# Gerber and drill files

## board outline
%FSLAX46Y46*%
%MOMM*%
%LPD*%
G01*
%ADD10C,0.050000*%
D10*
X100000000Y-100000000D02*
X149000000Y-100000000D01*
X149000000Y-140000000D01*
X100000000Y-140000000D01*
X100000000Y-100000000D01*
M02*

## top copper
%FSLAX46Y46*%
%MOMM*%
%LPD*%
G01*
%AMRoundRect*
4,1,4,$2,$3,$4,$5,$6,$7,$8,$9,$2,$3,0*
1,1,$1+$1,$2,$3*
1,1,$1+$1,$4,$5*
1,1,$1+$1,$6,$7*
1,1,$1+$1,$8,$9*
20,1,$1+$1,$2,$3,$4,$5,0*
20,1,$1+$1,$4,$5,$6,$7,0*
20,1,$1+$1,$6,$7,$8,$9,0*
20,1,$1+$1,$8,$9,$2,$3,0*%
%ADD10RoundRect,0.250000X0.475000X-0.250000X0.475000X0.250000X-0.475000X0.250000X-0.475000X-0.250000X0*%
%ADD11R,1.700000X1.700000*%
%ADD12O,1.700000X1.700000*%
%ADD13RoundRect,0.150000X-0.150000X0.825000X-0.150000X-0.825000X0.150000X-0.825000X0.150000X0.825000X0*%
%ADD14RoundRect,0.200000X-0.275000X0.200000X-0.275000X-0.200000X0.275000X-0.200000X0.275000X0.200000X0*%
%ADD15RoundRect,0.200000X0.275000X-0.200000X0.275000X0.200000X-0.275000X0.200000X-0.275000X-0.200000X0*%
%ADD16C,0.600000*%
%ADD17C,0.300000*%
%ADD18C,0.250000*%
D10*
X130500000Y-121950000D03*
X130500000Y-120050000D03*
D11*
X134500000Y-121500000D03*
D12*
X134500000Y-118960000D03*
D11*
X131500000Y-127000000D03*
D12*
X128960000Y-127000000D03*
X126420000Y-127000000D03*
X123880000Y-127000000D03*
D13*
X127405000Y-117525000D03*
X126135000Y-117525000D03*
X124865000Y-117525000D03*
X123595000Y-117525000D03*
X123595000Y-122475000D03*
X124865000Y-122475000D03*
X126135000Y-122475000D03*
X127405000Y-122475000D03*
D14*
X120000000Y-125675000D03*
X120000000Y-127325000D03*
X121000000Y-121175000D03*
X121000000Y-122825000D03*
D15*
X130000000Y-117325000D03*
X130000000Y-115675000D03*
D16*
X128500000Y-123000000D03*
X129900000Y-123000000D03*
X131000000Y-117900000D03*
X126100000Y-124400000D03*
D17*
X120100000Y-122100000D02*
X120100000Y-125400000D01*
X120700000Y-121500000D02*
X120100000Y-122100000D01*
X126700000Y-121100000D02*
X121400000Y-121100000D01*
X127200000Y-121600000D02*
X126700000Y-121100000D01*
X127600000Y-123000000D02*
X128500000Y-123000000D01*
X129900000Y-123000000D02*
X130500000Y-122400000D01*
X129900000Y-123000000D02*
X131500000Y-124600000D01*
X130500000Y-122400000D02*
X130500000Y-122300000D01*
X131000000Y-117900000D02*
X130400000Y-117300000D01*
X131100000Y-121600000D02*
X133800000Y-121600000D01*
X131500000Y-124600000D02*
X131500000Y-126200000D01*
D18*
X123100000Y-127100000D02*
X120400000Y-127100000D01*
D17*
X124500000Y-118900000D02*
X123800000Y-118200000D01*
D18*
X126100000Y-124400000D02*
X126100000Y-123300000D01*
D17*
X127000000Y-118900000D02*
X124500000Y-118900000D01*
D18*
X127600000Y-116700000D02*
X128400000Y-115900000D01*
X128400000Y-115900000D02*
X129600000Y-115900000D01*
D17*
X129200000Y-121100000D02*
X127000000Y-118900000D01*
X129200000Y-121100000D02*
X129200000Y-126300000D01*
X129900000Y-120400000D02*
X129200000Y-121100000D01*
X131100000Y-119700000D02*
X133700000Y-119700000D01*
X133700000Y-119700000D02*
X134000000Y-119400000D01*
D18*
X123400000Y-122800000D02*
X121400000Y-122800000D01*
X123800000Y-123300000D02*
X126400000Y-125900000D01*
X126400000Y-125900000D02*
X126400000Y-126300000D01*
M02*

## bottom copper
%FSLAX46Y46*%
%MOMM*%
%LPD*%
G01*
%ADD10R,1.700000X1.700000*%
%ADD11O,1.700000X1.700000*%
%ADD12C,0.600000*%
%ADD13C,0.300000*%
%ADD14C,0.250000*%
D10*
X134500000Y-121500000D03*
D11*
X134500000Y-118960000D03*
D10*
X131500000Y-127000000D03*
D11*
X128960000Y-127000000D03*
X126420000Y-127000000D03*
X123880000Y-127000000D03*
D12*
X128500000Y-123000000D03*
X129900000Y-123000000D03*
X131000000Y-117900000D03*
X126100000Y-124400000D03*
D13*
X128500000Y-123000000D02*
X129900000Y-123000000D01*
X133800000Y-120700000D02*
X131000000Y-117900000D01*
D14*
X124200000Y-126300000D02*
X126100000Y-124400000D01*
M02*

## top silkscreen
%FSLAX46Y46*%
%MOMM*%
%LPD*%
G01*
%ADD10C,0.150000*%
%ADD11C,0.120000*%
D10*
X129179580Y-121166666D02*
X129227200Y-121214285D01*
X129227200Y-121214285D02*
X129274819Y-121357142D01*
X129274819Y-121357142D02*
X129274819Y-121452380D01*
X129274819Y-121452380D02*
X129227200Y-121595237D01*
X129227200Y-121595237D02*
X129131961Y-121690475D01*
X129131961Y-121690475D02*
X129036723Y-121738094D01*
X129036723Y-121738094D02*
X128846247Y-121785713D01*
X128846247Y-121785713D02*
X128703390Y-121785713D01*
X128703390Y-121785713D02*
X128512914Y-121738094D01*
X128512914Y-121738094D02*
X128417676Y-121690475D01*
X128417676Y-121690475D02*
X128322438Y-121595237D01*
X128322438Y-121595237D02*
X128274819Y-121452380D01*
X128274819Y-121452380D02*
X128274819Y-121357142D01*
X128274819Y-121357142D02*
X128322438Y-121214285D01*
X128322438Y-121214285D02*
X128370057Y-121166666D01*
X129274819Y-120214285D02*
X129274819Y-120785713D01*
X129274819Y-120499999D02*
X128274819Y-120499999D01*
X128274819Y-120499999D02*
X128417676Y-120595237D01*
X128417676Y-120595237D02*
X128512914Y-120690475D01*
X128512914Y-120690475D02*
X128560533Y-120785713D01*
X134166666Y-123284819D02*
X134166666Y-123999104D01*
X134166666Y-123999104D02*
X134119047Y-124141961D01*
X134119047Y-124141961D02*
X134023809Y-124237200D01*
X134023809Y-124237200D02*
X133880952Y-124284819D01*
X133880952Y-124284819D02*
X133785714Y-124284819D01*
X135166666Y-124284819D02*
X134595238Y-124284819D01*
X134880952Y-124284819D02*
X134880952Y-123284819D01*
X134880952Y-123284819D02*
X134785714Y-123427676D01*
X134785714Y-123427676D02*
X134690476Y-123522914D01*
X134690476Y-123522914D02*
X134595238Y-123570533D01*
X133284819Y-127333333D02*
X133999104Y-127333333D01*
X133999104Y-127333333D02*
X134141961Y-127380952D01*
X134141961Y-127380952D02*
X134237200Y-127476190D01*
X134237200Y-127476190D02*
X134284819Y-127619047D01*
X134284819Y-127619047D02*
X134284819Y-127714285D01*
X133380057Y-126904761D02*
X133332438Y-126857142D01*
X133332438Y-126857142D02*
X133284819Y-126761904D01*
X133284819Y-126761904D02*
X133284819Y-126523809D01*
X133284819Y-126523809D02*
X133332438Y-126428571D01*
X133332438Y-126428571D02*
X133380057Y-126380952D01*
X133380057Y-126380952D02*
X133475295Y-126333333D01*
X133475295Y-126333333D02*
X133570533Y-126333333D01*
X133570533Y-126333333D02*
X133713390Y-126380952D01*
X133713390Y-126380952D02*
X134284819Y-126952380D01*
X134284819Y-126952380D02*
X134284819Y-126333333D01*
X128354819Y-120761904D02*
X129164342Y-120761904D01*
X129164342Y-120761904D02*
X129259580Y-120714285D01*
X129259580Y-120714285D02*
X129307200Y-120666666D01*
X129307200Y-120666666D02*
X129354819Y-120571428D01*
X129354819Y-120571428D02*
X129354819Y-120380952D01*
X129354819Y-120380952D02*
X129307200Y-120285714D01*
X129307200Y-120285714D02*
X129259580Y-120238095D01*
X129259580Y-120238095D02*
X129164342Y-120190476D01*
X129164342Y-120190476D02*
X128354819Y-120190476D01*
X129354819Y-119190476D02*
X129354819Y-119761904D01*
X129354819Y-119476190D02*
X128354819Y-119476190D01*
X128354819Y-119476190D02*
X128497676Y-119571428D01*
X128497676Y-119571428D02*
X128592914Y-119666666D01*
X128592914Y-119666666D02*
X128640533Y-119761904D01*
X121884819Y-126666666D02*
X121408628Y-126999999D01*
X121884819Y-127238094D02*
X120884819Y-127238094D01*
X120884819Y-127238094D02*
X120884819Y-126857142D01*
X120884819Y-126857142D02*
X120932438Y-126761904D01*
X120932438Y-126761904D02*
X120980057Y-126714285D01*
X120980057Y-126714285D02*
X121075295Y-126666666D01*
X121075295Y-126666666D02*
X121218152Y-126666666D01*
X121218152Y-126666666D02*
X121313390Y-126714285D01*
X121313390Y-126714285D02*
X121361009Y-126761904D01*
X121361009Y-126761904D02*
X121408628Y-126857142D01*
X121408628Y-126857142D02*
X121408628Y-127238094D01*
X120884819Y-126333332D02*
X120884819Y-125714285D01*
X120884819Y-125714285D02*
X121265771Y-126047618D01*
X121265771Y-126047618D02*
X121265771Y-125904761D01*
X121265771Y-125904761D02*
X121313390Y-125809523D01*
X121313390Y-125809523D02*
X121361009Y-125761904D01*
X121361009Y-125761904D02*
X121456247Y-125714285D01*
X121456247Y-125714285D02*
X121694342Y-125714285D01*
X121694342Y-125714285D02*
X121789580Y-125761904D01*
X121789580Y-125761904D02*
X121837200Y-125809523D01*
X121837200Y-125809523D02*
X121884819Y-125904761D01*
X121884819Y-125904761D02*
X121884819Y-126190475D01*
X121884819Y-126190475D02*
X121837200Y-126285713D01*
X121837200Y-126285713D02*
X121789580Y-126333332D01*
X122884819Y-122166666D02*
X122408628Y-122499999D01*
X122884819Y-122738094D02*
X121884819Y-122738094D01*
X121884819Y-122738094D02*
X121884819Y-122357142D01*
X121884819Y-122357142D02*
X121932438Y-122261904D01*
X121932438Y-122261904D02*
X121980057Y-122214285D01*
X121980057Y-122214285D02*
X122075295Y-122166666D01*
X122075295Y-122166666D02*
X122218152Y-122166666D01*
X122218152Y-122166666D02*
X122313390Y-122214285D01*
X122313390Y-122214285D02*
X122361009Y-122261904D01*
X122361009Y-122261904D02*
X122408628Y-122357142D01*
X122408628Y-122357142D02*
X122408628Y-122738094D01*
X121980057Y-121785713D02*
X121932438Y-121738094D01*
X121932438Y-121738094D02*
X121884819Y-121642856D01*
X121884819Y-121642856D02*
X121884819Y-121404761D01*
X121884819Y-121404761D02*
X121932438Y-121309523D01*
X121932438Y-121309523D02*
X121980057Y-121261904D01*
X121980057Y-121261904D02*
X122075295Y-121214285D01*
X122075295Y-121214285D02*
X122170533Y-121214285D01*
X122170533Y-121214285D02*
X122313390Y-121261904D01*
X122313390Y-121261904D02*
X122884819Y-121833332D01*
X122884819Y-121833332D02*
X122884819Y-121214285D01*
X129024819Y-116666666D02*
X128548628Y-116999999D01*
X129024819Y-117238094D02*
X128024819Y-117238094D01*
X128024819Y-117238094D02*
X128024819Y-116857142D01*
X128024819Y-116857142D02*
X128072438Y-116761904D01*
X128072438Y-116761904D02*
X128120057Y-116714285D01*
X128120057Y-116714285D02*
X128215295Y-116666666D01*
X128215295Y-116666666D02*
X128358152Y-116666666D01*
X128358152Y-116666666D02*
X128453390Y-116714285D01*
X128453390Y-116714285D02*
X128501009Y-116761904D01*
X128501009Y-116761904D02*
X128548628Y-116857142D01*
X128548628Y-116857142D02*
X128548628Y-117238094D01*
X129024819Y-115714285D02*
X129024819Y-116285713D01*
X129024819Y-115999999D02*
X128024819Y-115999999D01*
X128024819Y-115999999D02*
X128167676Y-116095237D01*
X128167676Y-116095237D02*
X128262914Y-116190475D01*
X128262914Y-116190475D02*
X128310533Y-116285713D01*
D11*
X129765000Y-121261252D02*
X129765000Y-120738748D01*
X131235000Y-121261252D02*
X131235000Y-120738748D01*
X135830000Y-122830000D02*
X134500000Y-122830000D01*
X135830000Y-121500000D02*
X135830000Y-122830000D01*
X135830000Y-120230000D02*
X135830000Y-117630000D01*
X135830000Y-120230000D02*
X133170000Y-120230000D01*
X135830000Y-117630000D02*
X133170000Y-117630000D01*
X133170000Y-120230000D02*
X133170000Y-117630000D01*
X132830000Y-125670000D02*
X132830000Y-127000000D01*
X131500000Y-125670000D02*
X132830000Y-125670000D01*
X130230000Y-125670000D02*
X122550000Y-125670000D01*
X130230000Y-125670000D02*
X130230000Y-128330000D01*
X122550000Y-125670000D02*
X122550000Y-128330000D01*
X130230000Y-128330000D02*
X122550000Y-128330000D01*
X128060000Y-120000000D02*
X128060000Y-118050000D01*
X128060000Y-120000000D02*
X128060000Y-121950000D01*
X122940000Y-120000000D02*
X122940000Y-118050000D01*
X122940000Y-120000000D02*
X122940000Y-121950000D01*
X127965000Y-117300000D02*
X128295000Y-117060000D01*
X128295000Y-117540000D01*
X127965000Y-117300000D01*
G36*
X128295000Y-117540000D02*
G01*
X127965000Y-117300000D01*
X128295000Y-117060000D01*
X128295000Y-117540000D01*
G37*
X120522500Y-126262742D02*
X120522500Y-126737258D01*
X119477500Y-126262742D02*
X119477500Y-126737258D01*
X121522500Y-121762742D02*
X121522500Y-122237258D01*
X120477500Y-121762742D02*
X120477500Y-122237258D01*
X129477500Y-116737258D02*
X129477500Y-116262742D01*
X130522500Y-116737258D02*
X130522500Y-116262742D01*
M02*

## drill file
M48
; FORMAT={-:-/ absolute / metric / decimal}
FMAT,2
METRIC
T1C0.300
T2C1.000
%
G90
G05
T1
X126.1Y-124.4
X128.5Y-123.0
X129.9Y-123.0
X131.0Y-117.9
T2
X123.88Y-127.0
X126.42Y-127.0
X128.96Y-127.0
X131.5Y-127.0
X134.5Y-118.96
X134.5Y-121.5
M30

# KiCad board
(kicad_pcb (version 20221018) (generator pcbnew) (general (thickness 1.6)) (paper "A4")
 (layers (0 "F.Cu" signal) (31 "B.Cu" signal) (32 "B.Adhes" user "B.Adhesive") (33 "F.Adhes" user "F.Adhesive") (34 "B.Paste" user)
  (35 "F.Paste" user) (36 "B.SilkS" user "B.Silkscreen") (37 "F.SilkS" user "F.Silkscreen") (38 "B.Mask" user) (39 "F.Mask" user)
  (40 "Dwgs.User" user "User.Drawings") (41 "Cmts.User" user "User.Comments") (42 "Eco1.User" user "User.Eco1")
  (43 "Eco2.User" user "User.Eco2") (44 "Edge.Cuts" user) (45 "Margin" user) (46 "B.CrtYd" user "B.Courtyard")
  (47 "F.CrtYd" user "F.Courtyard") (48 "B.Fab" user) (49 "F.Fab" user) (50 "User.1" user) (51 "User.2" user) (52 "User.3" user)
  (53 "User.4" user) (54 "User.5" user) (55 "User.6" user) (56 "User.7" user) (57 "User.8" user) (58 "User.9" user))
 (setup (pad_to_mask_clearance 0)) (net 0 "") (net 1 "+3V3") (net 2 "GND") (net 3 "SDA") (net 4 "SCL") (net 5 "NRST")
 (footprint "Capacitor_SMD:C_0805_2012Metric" (layer "F.Cu") (at 130.5 121 90)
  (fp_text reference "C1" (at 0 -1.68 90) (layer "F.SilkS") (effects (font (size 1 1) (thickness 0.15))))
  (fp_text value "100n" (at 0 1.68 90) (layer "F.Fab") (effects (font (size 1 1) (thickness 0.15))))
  (fp_line (start -0.261252 -0.735) (end 0.261252 -0.735) (stroke (width 0.12) (type solid)) (layer "F.SilkS"))
  (fp_line (start -0.261252 0.735) (end 0.261252 0.735) (stroke (width 0.12) (type solid)) (layer "F.SilkS"))
  (pad "1" smd roundrect (at -0.95 0 90) (size 1 1.45) (layers "F.Cu" "F.Paste" "F.Mask") (roundrect_rratio 0.25) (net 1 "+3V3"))
  (pad "2" smd roundrect (at 0.95 0 90) (size 1 1.45) (layers "F.Cu" "F.Paste" "F.Mask") (roundrect_rratio 0.25) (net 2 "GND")))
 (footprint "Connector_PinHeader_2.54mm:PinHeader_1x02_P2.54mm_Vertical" (layer "F.Cu") (at 134.5 121.5 180)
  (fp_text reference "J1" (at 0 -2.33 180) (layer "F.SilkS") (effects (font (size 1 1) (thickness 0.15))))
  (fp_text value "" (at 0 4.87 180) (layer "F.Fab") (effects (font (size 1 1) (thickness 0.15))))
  (fp_line (start -1.33 -1.33) (end 0 -1.33) (stroke (width 0.12) (type solid)) (layer "F.SilkS"))
  (fp_line (start -1.33 0) (end -1.33 -1.33) (stroke (width 0.12) (type solid)) (layer "F.SilkS"))
  (fp_line (start -1.33 1.27) (end -1.33 3.87) (stroke (width 0.12) (type solid)) (layer "F.SilkS"))
  (fp_line (start -1.33 1.27) (end 1.33 1.27) (stroke (width 0.12) (type solid)) (layer "F.SilkS"))
  (fp_line (start -1.33 3.87) (end 1.33 3.87) (stroke (width 0.12) (type solid)) (layer "F.SilkS"))
  (fp_line (start 1.33 1.27) (end 1.33 3.87) (stroke (width 0.12) (type solid)) (layer "F.SilkS"))
  (pad "1" thru_hole rect (at 0 0 180) (size 1.7 1.7) (drill 1) (layers "*.Cu" "*.Mask") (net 1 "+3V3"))
  (pad "2" thru_hole oval (at 0 2.54 180) (size 1.7 1.7) (drill 1) (layers "*.Cu" "*.Mask") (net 2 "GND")))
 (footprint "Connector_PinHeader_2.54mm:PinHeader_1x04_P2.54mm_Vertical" (layer "F.Cu") (at 131.5 127 -90)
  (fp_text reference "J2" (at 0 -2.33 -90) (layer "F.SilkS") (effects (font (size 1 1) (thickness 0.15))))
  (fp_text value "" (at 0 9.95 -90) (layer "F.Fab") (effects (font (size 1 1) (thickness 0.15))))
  (fp_line (start -1.33 -1.33) (end 0 -1.33) (stroke (width 0.12) (type solid)) (layer "F.SilkS"))
  (fp_line (start -1.33 0) (end -1.33 -1.33) (stroke (width 0.12) (type solid)) (layer "F.SilkS"))
  (fp_line (start -1.33 1.27) (end -1.33 8.95) (stroke (width 0.12) (type solid)) (layer "F.SilkS"))
  (fp_line (start -1.33 1.27) (end 1.33 1.27) (stroke (width 0.12) (type solid)) (layer "F.SilkS"))
  (fp_line (start -1.33 8.95) (end 1.33 8.95) (stroke (width 0.12) (type solid)) (layer "F.SilkS"))
  (fp_line (start 1.33 1.27) (end 1.33 8.95) (stroke (width 0.12) (type solid)) (layer "F.SilkS"))
  (pad "1" thru_hole rect (at 0 0 270) (size 1.7 1.7) (drill 1) (layers "*.Cu" "*.Mask") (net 1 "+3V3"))
  (pad "2" thru_hole oval (at 0 2.54 270) (size 1.7 1.7) (drill 1) (layers "*.Cu" "*.Mask") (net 2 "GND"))
  (pad "3" thru_hole oval (at 0 5.08 270) (size 1.7 1.7) (drill 1) (layers "*.Cu" "*.Mask") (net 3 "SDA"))
  (pad "4" thru_hole oval (at 0 7.62 270) (size 1.7 1.7) (drill 1) (layers "*.Cu" "*.Mask") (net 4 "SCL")))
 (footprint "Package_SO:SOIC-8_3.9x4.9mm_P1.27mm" (layer "F.Cu") (at 125.5 120 -90)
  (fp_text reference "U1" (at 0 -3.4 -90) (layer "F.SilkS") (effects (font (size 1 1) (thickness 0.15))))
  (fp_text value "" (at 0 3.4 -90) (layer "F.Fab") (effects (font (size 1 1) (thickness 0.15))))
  (fp_line (start 0 -2.56) (end -1.95 -2.56) (stroke (width 0.12) (type solid)) (layer "F.SilkS"))
  (fp_line (start 0 -2.56) (end 1.95 -2.56) (stroke (width 0.12) (type solid)) (layer "F.SilkS"))
  (fp_line (start 0 2.56) (end -1.95 2.56) (stroke (width 0.12) (type solid)) (layer "F.SilkS"))
  (fp_line (start 0 2.56) (end 1.95 2.56) (stroke (width 0.12) (type solid)) (layer "F.SilkS"))
  (fp_poly
   (pts (xy -2.7 -2.465) (xy -2.94 -2.795) (xy -2.46 -2.795) (xy -2.7 -2.465)) (stroke (width 0.12) (type solid)) (fill solid)
   (layer "F.SilkS"))
  (pad "1" smd roundrect (at -2.475 -1.905 270) (size 1.95 0.6) (layers "F.Cu" "F.Paste" "F.Mask") (roundrect_rratio 0.25) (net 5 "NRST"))
  (pad "2" smd roundrect (at -2.475 -0.635 270) (size 1.95 0.6) (layers "F.Cu" "F.Paste" "F.Mask") (roundrect_rratio 0.25))
  (pad "3" smd roundrect (at -2.475 0.635 270) (size 1.95 0.6) (layers "F.Cu" "F.Paste" "F.Mask") (roundrect_rratio 0.25))
  (pad "4" smd roundrect (at -2.475 1.905 270) (size 1.95 0.6) (layers "F.Cu" "F.Paste" "F.Mask") (roundrect_rratio 0.25) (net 2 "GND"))
  (pad "5" smd roundrect (at 2.475 1.905 270) (size 1.95 0.6) (layers "F.Cu" "F.Paste" "F.Mask") (roundrect_rratio 0.25) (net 3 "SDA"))
  (pad "6" smd roundrect (at 2.475 0.635 270) (size 1.95 0.6) (layers "F.Cu" "F.Paste" "F.Mask") (roundrect_rratio 0.25))
  (pad "7" smd roundrect (at 2.475 -0.635 270) (size 1.95 0.6) (layers "F.Cu" "F.Paste" "F.Mask") (roundrect_rratio 0.25) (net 4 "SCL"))
  (pad "8" smd roundrect (at 2.475 -1.905 270) (size 1.95 0.6) (layers "F.Cu" "F.Paste" "F.Mask") (roundrect_rratio 0.25) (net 1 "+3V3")))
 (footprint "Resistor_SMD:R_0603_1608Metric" (layer "F.Cu") (at 120 126.5 -90)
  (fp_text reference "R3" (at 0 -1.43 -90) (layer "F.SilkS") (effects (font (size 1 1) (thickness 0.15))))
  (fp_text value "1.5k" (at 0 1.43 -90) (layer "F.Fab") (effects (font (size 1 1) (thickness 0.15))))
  (fp_line (start -0.237258 -0.5225) (end 0.237258 -0.5225) (stroke (width 0.12) (type solid)) (layer "F.SilkS"))
  (fp_line (start -0.237258 0.5225) (end 0.237258 0.5225) (stroke (width 0.12) (type solid)) (layer "F.SilkS"))
  (pad "1" smd roundrect (at -0.825 0 270) (size 0.8 0.95) (layers "F.Cu" "F.Paste" "F.Mask") (roundrect_rratio 0.25) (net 1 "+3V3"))
  (pad "2" smd roundrect (at 0.825 0 270) (size 0.8 0.95) (layers "F.Cu" "F.Paste" "F.Mask") (roundrect_rratio 0.25) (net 4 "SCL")))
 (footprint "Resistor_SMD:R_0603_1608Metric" (layer "F.Cu") (at 121 122 -90)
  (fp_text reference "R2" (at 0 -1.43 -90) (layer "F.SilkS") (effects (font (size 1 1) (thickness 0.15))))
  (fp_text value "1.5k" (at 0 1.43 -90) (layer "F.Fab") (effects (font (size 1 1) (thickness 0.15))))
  (fp_line (start -0.237258 -0.5225) (end 0.237258 -0.5225) (stroke (width 0.12) (type solid)) (layer "F.SilkS"))
  (fp_line (start -0.237258 0.5225) (end 0.237258 0.5225) (stroke (width 0.12) (type solid)) (layer "F.SilkS"))
  (pad "1" smd roundrect (at -0.825 0 270) (size 0.8 0.95) (layers "F.Cu" "F.Paste" "F.Mask") (roundrect_rratio 0.25) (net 1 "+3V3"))
  (pad "2" smd roundrect (at 0.825 0 270) (size 0.8 0.95) (layers "F.Cu" "F.Paste" "F.Mask") (roundrect_rratio 0.25) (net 3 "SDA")))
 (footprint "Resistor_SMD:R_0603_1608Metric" (layer "F.Cu") (at 130 116.5 90)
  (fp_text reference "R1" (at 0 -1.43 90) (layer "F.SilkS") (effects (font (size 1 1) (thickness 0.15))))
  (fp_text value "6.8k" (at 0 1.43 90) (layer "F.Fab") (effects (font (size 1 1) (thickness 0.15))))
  (fp_line (start -0.237258 -0.5225) (end 0.237258 -0.5225) (stroke (width 0.12) (type solid)) (layer "F.SilkS"))
  (fp_line (start -0.237258 0.5225) (end 0.237258 0.5225) (stroke (width 0.12) (type solid)) (layer "F.SilkS"))
  (pad "1" smd roundrect (at -0.825 0 90) (size 0.8 0.95) (layers "F.Cu" "F.Paste" "F.Mask") (roundrect_rratio 0.25) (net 1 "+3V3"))
  (pad "2" smd roundrect (at 0.825 0 90) (size 0.8 0.95) (layers "F.Cu" "F.Paste" "F.Mask") (roundrect_rratio 0.25) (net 5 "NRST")))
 (gr_rect (start 100 100) (end 149 140) (stroke (width 0.05) (type default)) (fill none) (layer "Edge.Cuts"))
 (segment (start 120.1 122.1) (end 120.1 125.4) (width 0.3) (layer "F.Cu") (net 1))
 (segment (start 120.7 121.5) (end 120.1 122.1) (width 0.3) (layer "F.Cu") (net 1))
 (segment (start 126.7 121.1) (end 121.4 121.1) (width 0.3) (layer "F.Cu") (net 1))
 (segment (start 127.2 121.6) (end 126.7 121.1) (width 0.3) (layer "F.Cu") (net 1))
 (segment (start 127.6 123) (end 128.5 123) (width 0.3) (layer "F.Cu") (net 1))
 (segment (start 129.9 123) (end 130.5 122.4) (width 0.3) (layer "F.Cu") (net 1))
 (segment (start 129.9 123) (end 131.5 124.6) (width 0.3) (layer "F.Cu") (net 1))
 (segment (start 130.5 122.4) (end 130.5 122.3) (width 0.3) (layer "F.Cu") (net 1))
 (segment (start 131 117.9) (end 130.4 117.3) (width 0.3) (layer "F.Cu") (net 1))
 (segment (start 131.1 121.6) (end 133.8 121.6) (width 0.3) (layer "F.Cu") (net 1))
 (segment (start 131.5 124.6) (end 131.5 126.2) (width 0.3) (layer "F.Cu") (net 1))
 (via (at 128.5 123) (size 0.6) (drill 0.3) (layers "F.Cu" "B.Cu") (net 1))
 (via (at 129.9 123) (size 0.6) (drill 0.3) (layers "F.Cu" "B.Cu") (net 1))
 (via (at 131 117.9) (size 0.6) (drill 0.3) (layers "F.Cu" "B.Cu") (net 1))
 (segment (start 123.1 127.1) (end 120.4 127.1) (width 0.25) (layer "F.Cu") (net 4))
 (segment (start 124.5 118.9) (end 123.8 118.2) (width 0.3) (layer "F.Cu") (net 2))
 (segment (start 126.1 124.4) (end 126.1 123.3) (width 0.25) (layer "F.Cu") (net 4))
 (segment (start 127 118.9) (end 124.5 118.9) (width 0.3) (layer "F.Cu") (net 2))
 (segment (start 127.6 116.7) (end 128.4 115.9) (width 0.25) (layer "F.Cu") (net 5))
 (segment (start 128.4 115.9) (end 129.6 115.9) (width 0.25) (layer "F.Cu") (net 5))
 (segment (start 128.5 123) (end 129.9 123) (width 0.3) (layer "B.Cu") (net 1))
 (segment (start 129.2 121.1) (end 127 118.9) (width 0.3) (layer "F.Cu") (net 2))
 (segment (start 129.2 121.1) (end 129.2 126.3) (width 0.3) (layer "F.Cu") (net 2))
 (segment (start 129.9 120.4) (end 129.2 121.1) (width 0.3) (layer "F.Cu") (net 2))
 (segment (start 131.1 119.7) (end 133.7 119.7) (width 0.3) (layer "F.Cu") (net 2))
 (segment (start 133.7 119.7) (end 134 119.4) (width 0.3) (layer "F.Cu") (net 2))
 (segment (start 133.8 120.7) (end 131 117.9) (width 0.3) (layer "B.Cu") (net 1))
 (via (at 126.1 124.4) (size 0.6) (drill 0.3) (layers "F.Cu" "B.Cu") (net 4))
 (segment (start 123.4 122.8) (end 121.4 122.8) (width 0.25) (layer "F.Cu") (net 3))
 (segment (start 123.8 123.3) (end 126.4 125.9) (width 0.25) (layer "F.Cu") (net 3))
 (segment (start 124.2 126.3) (end 126.1 124.4) (width 0.25) (layer "B.Cu") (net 4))
 (segment (start 126.4 125.9) (end 126.4 126.3) (width 0.25) (layer "F.Cu") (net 3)))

